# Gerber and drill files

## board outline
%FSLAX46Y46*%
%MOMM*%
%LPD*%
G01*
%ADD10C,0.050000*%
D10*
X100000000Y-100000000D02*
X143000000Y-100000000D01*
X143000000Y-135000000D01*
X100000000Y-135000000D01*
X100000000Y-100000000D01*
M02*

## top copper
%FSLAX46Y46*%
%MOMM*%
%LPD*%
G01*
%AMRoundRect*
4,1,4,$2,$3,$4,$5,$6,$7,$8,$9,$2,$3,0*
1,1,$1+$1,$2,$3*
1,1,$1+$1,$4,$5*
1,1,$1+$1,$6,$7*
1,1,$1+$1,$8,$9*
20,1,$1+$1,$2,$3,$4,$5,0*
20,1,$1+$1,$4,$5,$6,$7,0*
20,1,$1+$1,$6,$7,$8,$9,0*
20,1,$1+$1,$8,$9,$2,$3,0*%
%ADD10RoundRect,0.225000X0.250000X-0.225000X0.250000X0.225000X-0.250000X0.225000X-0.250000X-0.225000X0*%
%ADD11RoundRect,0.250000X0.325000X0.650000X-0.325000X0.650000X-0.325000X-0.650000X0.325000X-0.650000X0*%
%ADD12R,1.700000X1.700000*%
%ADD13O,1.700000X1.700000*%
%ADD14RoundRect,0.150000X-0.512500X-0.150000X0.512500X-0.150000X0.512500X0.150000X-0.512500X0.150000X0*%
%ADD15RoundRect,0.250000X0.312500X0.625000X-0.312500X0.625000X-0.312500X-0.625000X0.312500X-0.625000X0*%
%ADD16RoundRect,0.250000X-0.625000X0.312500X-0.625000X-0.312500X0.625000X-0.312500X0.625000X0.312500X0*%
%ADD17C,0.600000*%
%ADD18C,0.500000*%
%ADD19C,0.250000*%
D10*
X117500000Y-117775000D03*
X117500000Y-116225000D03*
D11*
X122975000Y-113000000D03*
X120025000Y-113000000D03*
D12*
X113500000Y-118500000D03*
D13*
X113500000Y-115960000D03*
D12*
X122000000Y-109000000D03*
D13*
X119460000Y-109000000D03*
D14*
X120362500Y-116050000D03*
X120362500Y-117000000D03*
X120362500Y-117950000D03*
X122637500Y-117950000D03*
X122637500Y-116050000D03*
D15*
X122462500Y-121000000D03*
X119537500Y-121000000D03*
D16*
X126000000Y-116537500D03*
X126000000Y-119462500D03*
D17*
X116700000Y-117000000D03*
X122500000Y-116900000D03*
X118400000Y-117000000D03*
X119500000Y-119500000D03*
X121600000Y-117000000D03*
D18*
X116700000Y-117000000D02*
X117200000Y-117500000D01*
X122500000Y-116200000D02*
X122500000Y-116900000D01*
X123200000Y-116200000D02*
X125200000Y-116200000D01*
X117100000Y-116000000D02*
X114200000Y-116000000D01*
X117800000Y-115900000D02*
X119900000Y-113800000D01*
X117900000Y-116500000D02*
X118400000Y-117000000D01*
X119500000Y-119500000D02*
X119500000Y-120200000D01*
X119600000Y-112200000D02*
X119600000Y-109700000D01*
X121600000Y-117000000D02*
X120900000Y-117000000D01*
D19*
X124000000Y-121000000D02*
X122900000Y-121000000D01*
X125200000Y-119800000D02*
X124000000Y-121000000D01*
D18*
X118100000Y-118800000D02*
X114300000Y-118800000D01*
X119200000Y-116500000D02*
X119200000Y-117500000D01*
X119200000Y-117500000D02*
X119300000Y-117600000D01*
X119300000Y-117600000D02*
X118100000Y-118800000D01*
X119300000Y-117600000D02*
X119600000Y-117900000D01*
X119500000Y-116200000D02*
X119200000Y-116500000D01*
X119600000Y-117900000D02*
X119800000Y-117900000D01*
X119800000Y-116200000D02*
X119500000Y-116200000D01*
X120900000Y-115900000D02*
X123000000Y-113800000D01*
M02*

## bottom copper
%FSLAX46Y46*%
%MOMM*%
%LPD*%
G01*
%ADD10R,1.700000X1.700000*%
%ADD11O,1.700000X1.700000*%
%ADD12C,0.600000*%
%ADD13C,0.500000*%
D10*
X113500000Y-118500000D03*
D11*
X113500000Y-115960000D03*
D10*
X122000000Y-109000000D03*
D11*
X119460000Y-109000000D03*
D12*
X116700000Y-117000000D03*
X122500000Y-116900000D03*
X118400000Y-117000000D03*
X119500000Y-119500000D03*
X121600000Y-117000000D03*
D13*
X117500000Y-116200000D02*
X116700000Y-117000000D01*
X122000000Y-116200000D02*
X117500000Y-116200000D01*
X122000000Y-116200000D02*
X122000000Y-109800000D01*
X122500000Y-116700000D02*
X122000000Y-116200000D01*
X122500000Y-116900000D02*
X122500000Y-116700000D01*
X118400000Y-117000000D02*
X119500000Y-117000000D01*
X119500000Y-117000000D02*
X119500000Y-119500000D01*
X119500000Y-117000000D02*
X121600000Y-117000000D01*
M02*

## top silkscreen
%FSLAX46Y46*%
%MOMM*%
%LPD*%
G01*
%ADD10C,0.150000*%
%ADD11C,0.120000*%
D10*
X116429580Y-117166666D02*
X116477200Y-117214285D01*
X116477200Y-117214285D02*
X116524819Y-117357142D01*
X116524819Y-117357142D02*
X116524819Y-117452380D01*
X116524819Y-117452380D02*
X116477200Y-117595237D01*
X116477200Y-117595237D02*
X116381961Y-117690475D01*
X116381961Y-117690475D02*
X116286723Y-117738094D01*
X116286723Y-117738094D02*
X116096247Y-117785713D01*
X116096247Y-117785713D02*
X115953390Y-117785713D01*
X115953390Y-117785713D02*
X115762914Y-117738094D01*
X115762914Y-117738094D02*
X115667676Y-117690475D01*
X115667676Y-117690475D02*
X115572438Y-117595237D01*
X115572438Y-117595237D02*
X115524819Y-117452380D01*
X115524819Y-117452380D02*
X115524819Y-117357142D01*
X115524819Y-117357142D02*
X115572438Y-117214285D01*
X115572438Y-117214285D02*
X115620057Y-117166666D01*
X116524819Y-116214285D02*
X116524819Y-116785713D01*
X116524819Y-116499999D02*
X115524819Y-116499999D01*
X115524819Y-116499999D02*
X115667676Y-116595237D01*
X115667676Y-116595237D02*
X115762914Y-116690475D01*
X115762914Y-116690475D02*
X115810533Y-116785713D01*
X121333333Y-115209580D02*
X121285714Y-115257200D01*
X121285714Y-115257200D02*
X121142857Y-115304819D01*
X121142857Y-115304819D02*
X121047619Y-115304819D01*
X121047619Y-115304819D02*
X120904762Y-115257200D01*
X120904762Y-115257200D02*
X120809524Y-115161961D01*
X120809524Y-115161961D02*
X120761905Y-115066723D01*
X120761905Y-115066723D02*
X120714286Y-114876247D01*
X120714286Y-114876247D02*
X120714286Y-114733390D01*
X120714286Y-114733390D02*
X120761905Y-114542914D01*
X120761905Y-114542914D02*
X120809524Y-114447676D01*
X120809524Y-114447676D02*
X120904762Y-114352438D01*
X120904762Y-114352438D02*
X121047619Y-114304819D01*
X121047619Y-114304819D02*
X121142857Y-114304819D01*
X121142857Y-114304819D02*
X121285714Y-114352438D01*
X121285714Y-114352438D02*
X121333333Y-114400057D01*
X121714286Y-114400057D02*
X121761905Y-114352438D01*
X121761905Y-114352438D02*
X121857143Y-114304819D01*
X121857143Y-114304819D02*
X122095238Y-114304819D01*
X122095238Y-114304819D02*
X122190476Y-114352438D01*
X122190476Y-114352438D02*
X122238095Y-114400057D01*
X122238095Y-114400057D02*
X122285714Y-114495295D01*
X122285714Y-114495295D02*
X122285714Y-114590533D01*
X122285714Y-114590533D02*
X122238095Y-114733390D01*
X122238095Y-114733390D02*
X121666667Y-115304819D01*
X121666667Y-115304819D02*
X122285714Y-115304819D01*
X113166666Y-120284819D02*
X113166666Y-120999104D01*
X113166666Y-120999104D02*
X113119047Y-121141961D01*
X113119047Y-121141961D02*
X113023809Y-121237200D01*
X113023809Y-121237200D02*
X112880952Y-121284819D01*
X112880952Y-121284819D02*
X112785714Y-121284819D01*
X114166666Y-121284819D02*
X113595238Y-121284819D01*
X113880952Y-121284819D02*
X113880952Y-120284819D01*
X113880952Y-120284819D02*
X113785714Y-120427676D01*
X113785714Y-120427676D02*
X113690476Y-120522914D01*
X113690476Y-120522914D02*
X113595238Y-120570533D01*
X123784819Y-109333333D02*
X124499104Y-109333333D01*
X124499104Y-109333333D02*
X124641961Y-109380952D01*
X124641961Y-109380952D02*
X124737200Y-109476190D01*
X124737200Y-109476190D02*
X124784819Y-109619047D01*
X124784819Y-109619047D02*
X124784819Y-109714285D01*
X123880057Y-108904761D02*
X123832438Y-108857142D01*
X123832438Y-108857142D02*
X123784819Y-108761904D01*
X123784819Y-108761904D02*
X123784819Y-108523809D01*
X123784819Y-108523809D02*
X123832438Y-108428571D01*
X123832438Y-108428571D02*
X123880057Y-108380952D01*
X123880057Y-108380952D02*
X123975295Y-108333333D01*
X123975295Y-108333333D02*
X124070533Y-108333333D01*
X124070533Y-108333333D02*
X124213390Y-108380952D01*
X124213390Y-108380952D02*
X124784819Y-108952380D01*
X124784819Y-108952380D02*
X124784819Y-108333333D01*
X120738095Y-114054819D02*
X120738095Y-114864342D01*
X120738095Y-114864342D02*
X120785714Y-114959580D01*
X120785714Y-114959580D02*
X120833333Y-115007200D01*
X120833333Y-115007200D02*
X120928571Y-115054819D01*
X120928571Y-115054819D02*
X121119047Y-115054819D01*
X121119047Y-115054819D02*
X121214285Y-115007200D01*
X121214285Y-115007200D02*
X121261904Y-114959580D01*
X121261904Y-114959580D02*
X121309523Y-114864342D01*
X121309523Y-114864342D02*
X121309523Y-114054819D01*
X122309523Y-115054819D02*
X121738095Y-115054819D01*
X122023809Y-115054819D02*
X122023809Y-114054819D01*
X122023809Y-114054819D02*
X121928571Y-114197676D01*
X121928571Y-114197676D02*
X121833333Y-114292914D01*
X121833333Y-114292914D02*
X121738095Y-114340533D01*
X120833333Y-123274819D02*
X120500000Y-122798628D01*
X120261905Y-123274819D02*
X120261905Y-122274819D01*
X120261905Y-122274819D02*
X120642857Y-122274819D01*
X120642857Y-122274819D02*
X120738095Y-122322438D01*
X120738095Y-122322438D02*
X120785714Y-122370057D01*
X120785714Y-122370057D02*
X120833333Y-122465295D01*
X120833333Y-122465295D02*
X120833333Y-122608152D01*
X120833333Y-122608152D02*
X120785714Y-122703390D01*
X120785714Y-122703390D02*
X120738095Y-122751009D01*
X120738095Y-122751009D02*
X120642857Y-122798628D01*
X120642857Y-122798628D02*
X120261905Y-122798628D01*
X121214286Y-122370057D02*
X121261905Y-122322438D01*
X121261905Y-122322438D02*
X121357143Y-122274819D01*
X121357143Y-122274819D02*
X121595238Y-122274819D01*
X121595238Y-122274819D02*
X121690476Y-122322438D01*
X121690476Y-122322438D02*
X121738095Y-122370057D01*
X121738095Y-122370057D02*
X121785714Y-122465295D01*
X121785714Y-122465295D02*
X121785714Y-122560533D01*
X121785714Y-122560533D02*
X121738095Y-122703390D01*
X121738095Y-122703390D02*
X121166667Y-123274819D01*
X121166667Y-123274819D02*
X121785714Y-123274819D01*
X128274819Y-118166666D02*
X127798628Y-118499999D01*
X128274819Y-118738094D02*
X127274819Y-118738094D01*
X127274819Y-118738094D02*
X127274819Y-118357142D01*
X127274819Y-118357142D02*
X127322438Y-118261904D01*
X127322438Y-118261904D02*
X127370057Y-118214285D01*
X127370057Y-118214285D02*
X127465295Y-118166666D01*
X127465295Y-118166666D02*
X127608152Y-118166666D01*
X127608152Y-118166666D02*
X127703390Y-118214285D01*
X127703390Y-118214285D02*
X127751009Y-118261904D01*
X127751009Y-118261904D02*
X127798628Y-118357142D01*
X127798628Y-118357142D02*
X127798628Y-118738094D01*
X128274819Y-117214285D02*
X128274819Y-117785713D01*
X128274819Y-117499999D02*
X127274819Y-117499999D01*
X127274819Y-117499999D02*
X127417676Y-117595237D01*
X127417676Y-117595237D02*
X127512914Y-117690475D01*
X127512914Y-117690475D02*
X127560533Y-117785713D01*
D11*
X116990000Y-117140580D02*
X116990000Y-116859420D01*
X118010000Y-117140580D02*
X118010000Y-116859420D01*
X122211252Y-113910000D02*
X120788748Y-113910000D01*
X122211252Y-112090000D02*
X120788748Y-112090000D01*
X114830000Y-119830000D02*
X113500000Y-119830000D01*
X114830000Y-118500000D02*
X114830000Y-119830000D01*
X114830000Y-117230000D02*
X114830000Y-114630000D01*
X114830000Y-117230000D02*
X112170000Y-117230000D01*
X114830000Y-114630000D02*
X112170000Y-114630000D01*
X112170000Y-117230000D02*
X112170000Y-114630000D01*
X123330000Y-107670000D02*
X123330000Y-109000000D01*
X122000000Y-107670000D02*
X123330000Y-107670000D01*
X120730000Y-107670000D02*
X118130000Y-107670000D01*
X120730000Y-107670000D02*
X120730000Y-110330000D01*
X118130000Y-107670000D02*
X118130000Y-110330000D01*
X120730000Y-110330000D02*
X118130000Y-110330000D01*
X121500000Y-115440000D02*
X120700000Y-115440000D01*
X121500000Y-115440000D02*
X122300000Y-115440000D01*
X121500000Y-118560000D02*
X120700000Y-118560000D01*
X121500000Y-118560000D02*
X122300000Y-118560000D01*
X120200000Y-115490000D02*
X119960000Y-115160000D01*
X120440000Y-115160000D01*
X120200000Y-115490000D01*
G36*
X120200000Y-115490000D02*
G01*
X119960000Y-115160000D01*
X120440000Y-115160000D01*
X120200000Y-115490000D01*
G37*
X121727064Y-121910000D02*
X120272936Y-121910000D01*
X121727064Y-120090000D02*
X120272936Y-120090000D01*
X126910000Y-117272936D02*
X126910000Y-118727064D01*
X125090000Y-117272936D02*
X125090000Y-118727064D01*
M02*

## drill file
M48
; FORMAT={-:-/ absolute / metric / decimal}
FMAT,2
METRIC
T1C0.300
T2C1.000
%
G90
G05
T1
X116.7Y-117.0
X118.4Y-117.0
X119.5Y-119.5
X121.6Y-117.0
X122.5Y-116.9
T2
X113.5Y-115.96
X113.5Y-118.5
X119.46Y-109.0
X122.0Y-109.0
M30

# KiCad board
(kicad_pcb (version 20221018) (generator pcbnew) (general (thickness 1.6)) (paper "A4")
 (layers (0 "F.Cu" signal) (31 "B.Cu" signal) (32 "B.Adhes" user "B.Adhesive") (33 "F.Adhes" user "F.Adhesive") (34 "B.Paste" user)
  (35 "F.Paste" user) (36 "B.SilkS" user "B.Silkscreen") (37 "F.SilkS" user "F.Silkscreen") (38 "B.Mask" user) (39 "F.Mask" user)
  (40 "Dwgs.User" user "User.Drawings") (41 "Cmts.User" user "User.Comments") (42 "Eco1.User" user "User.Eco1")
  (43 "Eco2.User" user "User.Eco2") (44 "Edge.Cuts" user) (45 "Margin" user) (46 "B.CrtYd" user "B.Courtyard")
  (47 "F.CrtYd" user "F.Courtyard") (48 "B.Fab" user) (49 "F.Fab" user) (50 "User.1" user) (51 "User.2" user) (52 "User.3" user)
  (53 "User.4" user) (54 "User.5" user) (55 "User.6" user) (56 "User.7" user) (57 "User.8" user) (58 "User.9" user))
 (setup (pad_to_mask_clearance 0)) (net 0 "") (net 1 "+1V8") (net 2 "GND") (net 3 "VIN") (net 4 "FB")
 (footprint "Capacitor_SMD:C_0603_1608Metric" (layer "F.Cu") (at 117.5 117 90)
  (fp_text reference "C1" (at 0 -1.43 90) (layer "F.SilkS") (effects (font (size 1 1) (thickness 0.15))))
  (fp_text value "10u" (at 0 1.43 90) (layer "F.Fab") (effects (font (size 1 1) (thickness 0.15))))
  (fp_line (start -0.14058 -0.51) (end 0.14058 -0.51) (stroke (width 0.12) (type solid)) (layer "F.SilkS"))
  (fp_line (start -0.14058 0.51) (end 0.14058 0.51) (stroke (width 0.12) (type solid)) (layer "F.SilkS"))
  (pad "1" smd roundrect (at -0.775 0 90) (size 0.9 0.95) (layers "F.Cu" "F.Paste" "F.Mask") (roundrect_rratio 0.25) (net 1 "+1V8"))
  (pad "2" smd roundrect (at 0.775 0 90) (size 0.9 0.95) (layers "F.Cu" "F.Paste" "F.Mask") (roundrect_rratio 0.25) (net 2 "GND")))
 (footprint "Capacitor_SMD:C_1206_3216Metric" (layer "F.Cu") (at 121.5 113 180)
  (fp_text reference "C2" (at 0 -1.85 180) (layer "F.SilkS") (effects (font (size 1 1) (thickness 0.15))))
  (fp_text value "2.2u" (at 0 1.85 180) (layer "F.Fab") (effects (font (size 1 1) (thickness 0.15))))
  (fp_line (start -0.711252 -0.91) (end 0.711252 -0.91) (stroke (width 0.12) (type solid)) (layer "F.SilkS"))
  (fp_line (start -0.711252 0.91) (end 0.711252 0.91) (stroke (width 0.12) (type solid)) (layer "F.SilkS"))
  (pad "1" smd roundrect (at -1.475 0 180) (size 1.15 1.8) (layers "F.Cu" "F.Paste" "F.Mask") (roundrect_rratio 0.217391) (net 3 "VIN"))
  (pad "2" smd roundrect (at 1.475 0 180) (size 1.15 1.8) (layers "F.Cu" "F.Paste" "F.Mask") (roundrect_rratio 0.217391) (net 2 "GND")))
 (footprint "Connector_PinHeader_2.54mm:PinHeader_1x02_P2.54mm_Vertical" (layer "F.Cu") (at 113.5 118.5 180)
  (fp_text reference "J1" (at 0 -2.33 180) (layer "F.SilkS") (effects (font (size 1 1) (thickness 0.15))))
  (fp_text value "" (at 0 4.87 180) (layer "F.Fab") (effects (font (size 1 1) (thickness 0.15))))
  (fp_line (start -1.33 -1.33) (end 0 -1.33) (stroke (width 0.12) (type solid)) (layer "F.SilkS"))
  (fp_line (start -1.33 0) (end -1.33 -1.33) (stroke (width 0.12) (type solid)) (layer "F.SilkS"))
  (fp_line (start -1.33 1.27) (end -1.33 3.87) (stroke (width 0.12) (type solid)) (layer "F.SilkS"))
  (fp_line (start -1.33 1.27) (end 1.33 1.27) (stroke (width 0.12) (type solid)) (layer "F.SilkS"))
  (fp_line (start -1.33 3.87) (end 1.33 3.87) (stroke (width 0.12) (type solid)) (layer "F.SilkS"))
  (fp_line (start 1.33 1.27) (end 1.33 3.87) (stroke (width 0.12) (type solid)) (layer "F.SilkS"))
  (pad "1" thru_hole rect (at 0 0 180) (size 1.7 1.7) (drill 1) (layers "*.Cu" "*.Mask") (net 3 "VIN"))
  (pad "2" thru_hole oval (at 0 2.54 180) (size 1.7 1.7) (drill 1) (layers "*.Cu" "*.Mask") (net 2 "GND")))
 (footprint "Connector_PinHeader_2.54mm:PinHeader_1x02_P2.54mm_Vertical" (layer "F.Cu") (at 122 109 -90)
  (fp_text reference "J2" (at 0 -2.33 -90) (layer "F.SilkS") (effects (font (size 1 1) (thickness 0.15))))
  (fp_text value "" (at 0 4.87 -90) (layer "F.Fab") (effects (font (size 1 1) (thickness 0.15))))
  (fp_line (start -1.33 -1.33) (end 0 -1.33) (stroke (width 0.12) (type solid)) (layer "F.SilkS"))
  (fp_line (start -1.33 0) (end -1.33 -1.33) (stroke (width 0.12) (type solid)) (layer "F.SilkS"))
  (fp_line (start -1.33 1.27) (end -1.33 3.87) (stroke (width 0.12) (type solid)) (layer "F.SilkS"))
  (fp_line (start -1.33 1.27) (end 1.33 1.27) (stroke (width 0.12) (type solid)) (layer "F.SilkS"))
  (fp_line (start -1.33 3.87) (end 1.33 3.87) (stroke (width 0.12) (type solid)) (layer "F.SilkS"))
  (fp_line (start 1.33 1.27) (end 1.33 3.87) (stroke (width 0.12) (type solid)) (layer "F.SilkS"))
  (pad "1" thru_hole rect (at 0 0 270) (size 1.7 1.7) (drill 1) (layers "*.Cu" "*.Mask") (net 1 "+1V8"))
  (pad "2" thru_hole oval (at 0 2.54 270) (size 1.7 1.7) (drill 1) (layers "*.Cu" "*.Mask") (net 2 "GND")))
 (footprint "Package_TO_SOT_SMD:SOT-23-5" (layer "F.Cu") (at 121.5 117)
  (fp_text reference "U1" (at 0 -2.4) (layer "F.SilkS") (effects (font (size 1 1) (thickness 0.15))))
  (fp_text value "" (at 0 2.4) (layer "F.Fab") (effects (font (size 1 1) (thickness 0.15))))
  (fp_line (start 0 -1.56) (end -0.8 -1.56) (stroke (width 0.12) (type solid)) (layer "F.SilkS"))
  (fp_line (start 0 -1.56) (end 0.8 -1.56) (stroke (width 0.12) (type solid)) (layer "F.SilkS"))
  (fp_line (start 0 1.56) (end -0.8 1.56) (stroke (width 0.12) (type solid)) (layer "F.SilkS"))
  (fp_line (start 0 1.56) (end 0.8 1.56) (stroke (width 0.12) (type solid)) (layer "F.SilkS"))
  (fp_poly
   (pts (xy -1.3 -1.51) (xy -1.54 -1.84) (xy -1.06 -1.84) (xy -1.3 -1.51)) (stroke (width 0.12) (type solid)) (fill solid) (layer "F.SilkS"))
  (pad "1" smd roundrect (at -1.1375 -0.95) (size 1.325 0.6) (layers "F.Cu" "F.Paste" "F.Mask") (roundrect_rratio 0.25) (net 3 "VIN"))
  (pad "2" smd roundrect (at -1.1375 0) (size 1.325 0.6) (layers "F.Cu" "F.Paste" "F.Mask") (roundrect_rratio 0.25) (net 2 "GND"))
  (pad "3" smd roundrect (at -1.1375 0.95) (size 1.325 0.6) (layers "F.Cu" "F.Paste" "F.Mask") (roundrect_rratio 0.25) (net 3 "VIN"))
  (pad "4" smd roundrect (at 1.1375 0.95) (size 1.325 0.6) (layers "F.Cu" "F.Paste" "F.Mask") (roundrect_rratio 0.25))
  (pad "5" smd roundrect (at 1.1375 -0.95) (size 1.325 0.6) (layers "F.Cu" "F.Paste" "F.Mask") (roundrect_rratio 0.25) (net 1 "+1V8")))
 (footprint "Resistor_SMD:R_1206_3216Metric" (layer "F.Cu") (at 121 121 180)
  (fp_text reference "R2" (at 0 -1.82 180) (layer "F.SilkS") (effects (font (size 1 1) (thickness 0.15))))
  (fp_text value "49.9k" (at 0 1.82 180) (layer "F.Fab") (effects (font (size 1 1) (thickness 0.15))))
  (fp_line (start -0.727064 -0.91) (end 0.727064 -0.91) (stroke (width 0.12) (type solid)) (layer "F.SilkS"))
  (fp_line (start -0.727064 0.91) (end 0.727064 0.91) (stroke (width 0.12) (type solid)) (layer "F.SilkS"))
  (pad "1" smd roundrect (at -1.4625 0 180) (size 1.125 1.75) (layers "F.Cu" "F.Paste" "F.Mask") (roundrect_rratio 0.222222) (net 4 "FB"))
  (pad "2" smd roundrect (at 1.4625 0 180) (size 1.125 1.75) (layers "F.Cu" "F.Paste" "F.Mask") (roundrect_rratio 0.222222) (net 2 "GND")))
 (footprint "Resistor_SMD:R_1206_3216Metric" (layer "F.Cu") (at 126 118 -90)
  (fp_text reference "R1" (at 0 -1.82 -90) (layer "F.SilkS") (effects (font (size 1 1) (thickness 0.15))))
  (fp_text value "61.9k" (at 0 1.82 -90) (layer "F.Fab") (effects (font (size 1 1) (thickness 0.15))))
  (fp_line (start -0.727064 -0.91) (end 0.727064 -0.91) (stroke (width 0.12) (type solid)) (layer "F.SilkS"))
  (fp_line (start -0.727064 0.91) (end 0.727064 0.91) (stroke (width 0.12) (type solid)) (layer "F.SilkS"))
  (pad "1" smd roundrect (at -1.4625 0 270) (size 1.125 1.75) (layers "F.Cu" "F.Paste" "F.Mask") (roundrect_rratio 0.222222) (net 1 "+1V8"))
  (pad "2" smd roundrect (at 1.4625 0 270) (size 1.125 1.75) (layers "F.Cu" "F.Paste" "F.Mask") (roundrect_rratio 0.222222) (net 4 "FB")))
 (gr_rect (start 100 100) (end 143 135) (stroke (width 0.05) (type default)) (fill none) (layer "Edge.Cuts"))
 (segment (start 116.7 117) (end 117.2 117.5) (width 0.5) (layer "F.Cu") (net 1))
 (segment (start 122.5 116.2) (end 122.5 116.9) (width 0.5) (layer "F.Cu") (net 1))
 (segment (start 123.2 116.2) (end 125.2 116.2) (width 0.5) (layer "F.Cu") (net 1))
 (via (at 116.7 117) (size 0.6) (drill 0.3) (layers "F.Cu" "B.Cu") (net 1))
 (via (at 122.5 116.9) (size 0.6) (drill 0.3) (layers "F.Cu" "B.Cu") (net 1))
 (segment (start 117.1 116) (end 114.2 116) (width 0.5) (layer "F.Cu") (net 2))
 (segment (start 117.5 116.2) (end 116.7 117) (width 0.5) (layer "B.Cu") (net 1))
 (segment (start 117.8 115.9) (end 119.9 113.8) (width 0.5) (layer "F.Cu") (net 2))
 (segment (start 117.9 116.5) (end 118.4 117) (width 0.5) (layer "F.Cu") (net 2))
 (segment (start 119.5 119.5) (end 119.5 120.2) (width 0.5) (layer "F.Cu") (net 2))
 (segment (start 119.6 112.2) (end 119.6 109.7) (width 0.5) (layer "F.Cu") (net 2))
 (segment (start 121.6 117) (end 120.9 117) (width 0.5) (layer "F.Cu") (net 2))
 (segment (start 122 116.2) (end 117.5 116.2) (width 0.5) (layer "B.Cu") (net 1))
 (segment (start 122 116.2) (end 122 109.8) (width 0.5) (layer "B.Cu") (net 1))
 (segment (start 122.5 116.7) (end 122 116.2) (width 0.5) (layer "B.Cu") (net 1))
 (segment (start 122.5 116.9) (end 122.5 116.7) (width 0.5) (layer "B.Cu") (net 1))
 (segment (start 124 121) (end 122.9 121) (width 0.25) (layer "F.Cu") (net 4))
 (segment (start 125.2 119.8) (end 124 121) (width 0.25) (layer "F.Cu") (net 4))
 (via (at 118.4 117) (size 0.6) (drill 0.3) (layers "F.Cu" "B.Cu") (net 2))
 (via (at 119.5 119.5) (size 0.6) (drill 0.3) (layers "F.Cu" "B.Cu") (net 2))
 (via (at 121.6 117) (size 0.6) (drill 0.3) (layers "F.Cu" "B.Cu") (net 2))
 (segment (start 118.1 118.8) (end 114.3 118.8) (width 0.5) (layer "F.Cu") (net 3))
 (segment (start 118.4 117) (end 119.5 117) (width 0.5) (layer "B.Cu") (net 2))
 (segment (start 119.2 116.5) (end 119.2 117.5) (width 0.5) (layer "F.Cu") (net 3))
 (segment (start 119.2 117.5) (end 119.3 117.6) (width 0.5) (layer "F.Cu") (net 3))
 (segment (start 119.3 117.6) (end 118.1 118.8) (width 0.5) (layer "F.Cu") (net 3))
 (segment (start 119.3 117.6) (end 119.6 117.9) (width 0.5) (layer "F.Cu") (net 3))
 (segment (start 119.5 116.2) (end 119.2 116.5) (width 0.5) (layer "F.Cu") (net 3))
 (segment (start 119.5 117) (end 119.5 119.5) (width 0.5) (layer "B.Cu") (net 2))
 (segment (start 119.5 117) (end 121.6 117) (width 0.5) (layer "B.Cu") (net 2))
 (segment (start 119.6 117.9) (end 119.8 117.9) (width 0.5) (layer "F.Cu") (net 3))
 (segment (start 119.8 116.2) (end 119.5 116.2) (width 0.5) (layer "F.Cu") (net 3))
 (segment (start 120.9 115.9) (end 123 113.8) (width 0.5) (layer "F.Cu") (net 3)))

